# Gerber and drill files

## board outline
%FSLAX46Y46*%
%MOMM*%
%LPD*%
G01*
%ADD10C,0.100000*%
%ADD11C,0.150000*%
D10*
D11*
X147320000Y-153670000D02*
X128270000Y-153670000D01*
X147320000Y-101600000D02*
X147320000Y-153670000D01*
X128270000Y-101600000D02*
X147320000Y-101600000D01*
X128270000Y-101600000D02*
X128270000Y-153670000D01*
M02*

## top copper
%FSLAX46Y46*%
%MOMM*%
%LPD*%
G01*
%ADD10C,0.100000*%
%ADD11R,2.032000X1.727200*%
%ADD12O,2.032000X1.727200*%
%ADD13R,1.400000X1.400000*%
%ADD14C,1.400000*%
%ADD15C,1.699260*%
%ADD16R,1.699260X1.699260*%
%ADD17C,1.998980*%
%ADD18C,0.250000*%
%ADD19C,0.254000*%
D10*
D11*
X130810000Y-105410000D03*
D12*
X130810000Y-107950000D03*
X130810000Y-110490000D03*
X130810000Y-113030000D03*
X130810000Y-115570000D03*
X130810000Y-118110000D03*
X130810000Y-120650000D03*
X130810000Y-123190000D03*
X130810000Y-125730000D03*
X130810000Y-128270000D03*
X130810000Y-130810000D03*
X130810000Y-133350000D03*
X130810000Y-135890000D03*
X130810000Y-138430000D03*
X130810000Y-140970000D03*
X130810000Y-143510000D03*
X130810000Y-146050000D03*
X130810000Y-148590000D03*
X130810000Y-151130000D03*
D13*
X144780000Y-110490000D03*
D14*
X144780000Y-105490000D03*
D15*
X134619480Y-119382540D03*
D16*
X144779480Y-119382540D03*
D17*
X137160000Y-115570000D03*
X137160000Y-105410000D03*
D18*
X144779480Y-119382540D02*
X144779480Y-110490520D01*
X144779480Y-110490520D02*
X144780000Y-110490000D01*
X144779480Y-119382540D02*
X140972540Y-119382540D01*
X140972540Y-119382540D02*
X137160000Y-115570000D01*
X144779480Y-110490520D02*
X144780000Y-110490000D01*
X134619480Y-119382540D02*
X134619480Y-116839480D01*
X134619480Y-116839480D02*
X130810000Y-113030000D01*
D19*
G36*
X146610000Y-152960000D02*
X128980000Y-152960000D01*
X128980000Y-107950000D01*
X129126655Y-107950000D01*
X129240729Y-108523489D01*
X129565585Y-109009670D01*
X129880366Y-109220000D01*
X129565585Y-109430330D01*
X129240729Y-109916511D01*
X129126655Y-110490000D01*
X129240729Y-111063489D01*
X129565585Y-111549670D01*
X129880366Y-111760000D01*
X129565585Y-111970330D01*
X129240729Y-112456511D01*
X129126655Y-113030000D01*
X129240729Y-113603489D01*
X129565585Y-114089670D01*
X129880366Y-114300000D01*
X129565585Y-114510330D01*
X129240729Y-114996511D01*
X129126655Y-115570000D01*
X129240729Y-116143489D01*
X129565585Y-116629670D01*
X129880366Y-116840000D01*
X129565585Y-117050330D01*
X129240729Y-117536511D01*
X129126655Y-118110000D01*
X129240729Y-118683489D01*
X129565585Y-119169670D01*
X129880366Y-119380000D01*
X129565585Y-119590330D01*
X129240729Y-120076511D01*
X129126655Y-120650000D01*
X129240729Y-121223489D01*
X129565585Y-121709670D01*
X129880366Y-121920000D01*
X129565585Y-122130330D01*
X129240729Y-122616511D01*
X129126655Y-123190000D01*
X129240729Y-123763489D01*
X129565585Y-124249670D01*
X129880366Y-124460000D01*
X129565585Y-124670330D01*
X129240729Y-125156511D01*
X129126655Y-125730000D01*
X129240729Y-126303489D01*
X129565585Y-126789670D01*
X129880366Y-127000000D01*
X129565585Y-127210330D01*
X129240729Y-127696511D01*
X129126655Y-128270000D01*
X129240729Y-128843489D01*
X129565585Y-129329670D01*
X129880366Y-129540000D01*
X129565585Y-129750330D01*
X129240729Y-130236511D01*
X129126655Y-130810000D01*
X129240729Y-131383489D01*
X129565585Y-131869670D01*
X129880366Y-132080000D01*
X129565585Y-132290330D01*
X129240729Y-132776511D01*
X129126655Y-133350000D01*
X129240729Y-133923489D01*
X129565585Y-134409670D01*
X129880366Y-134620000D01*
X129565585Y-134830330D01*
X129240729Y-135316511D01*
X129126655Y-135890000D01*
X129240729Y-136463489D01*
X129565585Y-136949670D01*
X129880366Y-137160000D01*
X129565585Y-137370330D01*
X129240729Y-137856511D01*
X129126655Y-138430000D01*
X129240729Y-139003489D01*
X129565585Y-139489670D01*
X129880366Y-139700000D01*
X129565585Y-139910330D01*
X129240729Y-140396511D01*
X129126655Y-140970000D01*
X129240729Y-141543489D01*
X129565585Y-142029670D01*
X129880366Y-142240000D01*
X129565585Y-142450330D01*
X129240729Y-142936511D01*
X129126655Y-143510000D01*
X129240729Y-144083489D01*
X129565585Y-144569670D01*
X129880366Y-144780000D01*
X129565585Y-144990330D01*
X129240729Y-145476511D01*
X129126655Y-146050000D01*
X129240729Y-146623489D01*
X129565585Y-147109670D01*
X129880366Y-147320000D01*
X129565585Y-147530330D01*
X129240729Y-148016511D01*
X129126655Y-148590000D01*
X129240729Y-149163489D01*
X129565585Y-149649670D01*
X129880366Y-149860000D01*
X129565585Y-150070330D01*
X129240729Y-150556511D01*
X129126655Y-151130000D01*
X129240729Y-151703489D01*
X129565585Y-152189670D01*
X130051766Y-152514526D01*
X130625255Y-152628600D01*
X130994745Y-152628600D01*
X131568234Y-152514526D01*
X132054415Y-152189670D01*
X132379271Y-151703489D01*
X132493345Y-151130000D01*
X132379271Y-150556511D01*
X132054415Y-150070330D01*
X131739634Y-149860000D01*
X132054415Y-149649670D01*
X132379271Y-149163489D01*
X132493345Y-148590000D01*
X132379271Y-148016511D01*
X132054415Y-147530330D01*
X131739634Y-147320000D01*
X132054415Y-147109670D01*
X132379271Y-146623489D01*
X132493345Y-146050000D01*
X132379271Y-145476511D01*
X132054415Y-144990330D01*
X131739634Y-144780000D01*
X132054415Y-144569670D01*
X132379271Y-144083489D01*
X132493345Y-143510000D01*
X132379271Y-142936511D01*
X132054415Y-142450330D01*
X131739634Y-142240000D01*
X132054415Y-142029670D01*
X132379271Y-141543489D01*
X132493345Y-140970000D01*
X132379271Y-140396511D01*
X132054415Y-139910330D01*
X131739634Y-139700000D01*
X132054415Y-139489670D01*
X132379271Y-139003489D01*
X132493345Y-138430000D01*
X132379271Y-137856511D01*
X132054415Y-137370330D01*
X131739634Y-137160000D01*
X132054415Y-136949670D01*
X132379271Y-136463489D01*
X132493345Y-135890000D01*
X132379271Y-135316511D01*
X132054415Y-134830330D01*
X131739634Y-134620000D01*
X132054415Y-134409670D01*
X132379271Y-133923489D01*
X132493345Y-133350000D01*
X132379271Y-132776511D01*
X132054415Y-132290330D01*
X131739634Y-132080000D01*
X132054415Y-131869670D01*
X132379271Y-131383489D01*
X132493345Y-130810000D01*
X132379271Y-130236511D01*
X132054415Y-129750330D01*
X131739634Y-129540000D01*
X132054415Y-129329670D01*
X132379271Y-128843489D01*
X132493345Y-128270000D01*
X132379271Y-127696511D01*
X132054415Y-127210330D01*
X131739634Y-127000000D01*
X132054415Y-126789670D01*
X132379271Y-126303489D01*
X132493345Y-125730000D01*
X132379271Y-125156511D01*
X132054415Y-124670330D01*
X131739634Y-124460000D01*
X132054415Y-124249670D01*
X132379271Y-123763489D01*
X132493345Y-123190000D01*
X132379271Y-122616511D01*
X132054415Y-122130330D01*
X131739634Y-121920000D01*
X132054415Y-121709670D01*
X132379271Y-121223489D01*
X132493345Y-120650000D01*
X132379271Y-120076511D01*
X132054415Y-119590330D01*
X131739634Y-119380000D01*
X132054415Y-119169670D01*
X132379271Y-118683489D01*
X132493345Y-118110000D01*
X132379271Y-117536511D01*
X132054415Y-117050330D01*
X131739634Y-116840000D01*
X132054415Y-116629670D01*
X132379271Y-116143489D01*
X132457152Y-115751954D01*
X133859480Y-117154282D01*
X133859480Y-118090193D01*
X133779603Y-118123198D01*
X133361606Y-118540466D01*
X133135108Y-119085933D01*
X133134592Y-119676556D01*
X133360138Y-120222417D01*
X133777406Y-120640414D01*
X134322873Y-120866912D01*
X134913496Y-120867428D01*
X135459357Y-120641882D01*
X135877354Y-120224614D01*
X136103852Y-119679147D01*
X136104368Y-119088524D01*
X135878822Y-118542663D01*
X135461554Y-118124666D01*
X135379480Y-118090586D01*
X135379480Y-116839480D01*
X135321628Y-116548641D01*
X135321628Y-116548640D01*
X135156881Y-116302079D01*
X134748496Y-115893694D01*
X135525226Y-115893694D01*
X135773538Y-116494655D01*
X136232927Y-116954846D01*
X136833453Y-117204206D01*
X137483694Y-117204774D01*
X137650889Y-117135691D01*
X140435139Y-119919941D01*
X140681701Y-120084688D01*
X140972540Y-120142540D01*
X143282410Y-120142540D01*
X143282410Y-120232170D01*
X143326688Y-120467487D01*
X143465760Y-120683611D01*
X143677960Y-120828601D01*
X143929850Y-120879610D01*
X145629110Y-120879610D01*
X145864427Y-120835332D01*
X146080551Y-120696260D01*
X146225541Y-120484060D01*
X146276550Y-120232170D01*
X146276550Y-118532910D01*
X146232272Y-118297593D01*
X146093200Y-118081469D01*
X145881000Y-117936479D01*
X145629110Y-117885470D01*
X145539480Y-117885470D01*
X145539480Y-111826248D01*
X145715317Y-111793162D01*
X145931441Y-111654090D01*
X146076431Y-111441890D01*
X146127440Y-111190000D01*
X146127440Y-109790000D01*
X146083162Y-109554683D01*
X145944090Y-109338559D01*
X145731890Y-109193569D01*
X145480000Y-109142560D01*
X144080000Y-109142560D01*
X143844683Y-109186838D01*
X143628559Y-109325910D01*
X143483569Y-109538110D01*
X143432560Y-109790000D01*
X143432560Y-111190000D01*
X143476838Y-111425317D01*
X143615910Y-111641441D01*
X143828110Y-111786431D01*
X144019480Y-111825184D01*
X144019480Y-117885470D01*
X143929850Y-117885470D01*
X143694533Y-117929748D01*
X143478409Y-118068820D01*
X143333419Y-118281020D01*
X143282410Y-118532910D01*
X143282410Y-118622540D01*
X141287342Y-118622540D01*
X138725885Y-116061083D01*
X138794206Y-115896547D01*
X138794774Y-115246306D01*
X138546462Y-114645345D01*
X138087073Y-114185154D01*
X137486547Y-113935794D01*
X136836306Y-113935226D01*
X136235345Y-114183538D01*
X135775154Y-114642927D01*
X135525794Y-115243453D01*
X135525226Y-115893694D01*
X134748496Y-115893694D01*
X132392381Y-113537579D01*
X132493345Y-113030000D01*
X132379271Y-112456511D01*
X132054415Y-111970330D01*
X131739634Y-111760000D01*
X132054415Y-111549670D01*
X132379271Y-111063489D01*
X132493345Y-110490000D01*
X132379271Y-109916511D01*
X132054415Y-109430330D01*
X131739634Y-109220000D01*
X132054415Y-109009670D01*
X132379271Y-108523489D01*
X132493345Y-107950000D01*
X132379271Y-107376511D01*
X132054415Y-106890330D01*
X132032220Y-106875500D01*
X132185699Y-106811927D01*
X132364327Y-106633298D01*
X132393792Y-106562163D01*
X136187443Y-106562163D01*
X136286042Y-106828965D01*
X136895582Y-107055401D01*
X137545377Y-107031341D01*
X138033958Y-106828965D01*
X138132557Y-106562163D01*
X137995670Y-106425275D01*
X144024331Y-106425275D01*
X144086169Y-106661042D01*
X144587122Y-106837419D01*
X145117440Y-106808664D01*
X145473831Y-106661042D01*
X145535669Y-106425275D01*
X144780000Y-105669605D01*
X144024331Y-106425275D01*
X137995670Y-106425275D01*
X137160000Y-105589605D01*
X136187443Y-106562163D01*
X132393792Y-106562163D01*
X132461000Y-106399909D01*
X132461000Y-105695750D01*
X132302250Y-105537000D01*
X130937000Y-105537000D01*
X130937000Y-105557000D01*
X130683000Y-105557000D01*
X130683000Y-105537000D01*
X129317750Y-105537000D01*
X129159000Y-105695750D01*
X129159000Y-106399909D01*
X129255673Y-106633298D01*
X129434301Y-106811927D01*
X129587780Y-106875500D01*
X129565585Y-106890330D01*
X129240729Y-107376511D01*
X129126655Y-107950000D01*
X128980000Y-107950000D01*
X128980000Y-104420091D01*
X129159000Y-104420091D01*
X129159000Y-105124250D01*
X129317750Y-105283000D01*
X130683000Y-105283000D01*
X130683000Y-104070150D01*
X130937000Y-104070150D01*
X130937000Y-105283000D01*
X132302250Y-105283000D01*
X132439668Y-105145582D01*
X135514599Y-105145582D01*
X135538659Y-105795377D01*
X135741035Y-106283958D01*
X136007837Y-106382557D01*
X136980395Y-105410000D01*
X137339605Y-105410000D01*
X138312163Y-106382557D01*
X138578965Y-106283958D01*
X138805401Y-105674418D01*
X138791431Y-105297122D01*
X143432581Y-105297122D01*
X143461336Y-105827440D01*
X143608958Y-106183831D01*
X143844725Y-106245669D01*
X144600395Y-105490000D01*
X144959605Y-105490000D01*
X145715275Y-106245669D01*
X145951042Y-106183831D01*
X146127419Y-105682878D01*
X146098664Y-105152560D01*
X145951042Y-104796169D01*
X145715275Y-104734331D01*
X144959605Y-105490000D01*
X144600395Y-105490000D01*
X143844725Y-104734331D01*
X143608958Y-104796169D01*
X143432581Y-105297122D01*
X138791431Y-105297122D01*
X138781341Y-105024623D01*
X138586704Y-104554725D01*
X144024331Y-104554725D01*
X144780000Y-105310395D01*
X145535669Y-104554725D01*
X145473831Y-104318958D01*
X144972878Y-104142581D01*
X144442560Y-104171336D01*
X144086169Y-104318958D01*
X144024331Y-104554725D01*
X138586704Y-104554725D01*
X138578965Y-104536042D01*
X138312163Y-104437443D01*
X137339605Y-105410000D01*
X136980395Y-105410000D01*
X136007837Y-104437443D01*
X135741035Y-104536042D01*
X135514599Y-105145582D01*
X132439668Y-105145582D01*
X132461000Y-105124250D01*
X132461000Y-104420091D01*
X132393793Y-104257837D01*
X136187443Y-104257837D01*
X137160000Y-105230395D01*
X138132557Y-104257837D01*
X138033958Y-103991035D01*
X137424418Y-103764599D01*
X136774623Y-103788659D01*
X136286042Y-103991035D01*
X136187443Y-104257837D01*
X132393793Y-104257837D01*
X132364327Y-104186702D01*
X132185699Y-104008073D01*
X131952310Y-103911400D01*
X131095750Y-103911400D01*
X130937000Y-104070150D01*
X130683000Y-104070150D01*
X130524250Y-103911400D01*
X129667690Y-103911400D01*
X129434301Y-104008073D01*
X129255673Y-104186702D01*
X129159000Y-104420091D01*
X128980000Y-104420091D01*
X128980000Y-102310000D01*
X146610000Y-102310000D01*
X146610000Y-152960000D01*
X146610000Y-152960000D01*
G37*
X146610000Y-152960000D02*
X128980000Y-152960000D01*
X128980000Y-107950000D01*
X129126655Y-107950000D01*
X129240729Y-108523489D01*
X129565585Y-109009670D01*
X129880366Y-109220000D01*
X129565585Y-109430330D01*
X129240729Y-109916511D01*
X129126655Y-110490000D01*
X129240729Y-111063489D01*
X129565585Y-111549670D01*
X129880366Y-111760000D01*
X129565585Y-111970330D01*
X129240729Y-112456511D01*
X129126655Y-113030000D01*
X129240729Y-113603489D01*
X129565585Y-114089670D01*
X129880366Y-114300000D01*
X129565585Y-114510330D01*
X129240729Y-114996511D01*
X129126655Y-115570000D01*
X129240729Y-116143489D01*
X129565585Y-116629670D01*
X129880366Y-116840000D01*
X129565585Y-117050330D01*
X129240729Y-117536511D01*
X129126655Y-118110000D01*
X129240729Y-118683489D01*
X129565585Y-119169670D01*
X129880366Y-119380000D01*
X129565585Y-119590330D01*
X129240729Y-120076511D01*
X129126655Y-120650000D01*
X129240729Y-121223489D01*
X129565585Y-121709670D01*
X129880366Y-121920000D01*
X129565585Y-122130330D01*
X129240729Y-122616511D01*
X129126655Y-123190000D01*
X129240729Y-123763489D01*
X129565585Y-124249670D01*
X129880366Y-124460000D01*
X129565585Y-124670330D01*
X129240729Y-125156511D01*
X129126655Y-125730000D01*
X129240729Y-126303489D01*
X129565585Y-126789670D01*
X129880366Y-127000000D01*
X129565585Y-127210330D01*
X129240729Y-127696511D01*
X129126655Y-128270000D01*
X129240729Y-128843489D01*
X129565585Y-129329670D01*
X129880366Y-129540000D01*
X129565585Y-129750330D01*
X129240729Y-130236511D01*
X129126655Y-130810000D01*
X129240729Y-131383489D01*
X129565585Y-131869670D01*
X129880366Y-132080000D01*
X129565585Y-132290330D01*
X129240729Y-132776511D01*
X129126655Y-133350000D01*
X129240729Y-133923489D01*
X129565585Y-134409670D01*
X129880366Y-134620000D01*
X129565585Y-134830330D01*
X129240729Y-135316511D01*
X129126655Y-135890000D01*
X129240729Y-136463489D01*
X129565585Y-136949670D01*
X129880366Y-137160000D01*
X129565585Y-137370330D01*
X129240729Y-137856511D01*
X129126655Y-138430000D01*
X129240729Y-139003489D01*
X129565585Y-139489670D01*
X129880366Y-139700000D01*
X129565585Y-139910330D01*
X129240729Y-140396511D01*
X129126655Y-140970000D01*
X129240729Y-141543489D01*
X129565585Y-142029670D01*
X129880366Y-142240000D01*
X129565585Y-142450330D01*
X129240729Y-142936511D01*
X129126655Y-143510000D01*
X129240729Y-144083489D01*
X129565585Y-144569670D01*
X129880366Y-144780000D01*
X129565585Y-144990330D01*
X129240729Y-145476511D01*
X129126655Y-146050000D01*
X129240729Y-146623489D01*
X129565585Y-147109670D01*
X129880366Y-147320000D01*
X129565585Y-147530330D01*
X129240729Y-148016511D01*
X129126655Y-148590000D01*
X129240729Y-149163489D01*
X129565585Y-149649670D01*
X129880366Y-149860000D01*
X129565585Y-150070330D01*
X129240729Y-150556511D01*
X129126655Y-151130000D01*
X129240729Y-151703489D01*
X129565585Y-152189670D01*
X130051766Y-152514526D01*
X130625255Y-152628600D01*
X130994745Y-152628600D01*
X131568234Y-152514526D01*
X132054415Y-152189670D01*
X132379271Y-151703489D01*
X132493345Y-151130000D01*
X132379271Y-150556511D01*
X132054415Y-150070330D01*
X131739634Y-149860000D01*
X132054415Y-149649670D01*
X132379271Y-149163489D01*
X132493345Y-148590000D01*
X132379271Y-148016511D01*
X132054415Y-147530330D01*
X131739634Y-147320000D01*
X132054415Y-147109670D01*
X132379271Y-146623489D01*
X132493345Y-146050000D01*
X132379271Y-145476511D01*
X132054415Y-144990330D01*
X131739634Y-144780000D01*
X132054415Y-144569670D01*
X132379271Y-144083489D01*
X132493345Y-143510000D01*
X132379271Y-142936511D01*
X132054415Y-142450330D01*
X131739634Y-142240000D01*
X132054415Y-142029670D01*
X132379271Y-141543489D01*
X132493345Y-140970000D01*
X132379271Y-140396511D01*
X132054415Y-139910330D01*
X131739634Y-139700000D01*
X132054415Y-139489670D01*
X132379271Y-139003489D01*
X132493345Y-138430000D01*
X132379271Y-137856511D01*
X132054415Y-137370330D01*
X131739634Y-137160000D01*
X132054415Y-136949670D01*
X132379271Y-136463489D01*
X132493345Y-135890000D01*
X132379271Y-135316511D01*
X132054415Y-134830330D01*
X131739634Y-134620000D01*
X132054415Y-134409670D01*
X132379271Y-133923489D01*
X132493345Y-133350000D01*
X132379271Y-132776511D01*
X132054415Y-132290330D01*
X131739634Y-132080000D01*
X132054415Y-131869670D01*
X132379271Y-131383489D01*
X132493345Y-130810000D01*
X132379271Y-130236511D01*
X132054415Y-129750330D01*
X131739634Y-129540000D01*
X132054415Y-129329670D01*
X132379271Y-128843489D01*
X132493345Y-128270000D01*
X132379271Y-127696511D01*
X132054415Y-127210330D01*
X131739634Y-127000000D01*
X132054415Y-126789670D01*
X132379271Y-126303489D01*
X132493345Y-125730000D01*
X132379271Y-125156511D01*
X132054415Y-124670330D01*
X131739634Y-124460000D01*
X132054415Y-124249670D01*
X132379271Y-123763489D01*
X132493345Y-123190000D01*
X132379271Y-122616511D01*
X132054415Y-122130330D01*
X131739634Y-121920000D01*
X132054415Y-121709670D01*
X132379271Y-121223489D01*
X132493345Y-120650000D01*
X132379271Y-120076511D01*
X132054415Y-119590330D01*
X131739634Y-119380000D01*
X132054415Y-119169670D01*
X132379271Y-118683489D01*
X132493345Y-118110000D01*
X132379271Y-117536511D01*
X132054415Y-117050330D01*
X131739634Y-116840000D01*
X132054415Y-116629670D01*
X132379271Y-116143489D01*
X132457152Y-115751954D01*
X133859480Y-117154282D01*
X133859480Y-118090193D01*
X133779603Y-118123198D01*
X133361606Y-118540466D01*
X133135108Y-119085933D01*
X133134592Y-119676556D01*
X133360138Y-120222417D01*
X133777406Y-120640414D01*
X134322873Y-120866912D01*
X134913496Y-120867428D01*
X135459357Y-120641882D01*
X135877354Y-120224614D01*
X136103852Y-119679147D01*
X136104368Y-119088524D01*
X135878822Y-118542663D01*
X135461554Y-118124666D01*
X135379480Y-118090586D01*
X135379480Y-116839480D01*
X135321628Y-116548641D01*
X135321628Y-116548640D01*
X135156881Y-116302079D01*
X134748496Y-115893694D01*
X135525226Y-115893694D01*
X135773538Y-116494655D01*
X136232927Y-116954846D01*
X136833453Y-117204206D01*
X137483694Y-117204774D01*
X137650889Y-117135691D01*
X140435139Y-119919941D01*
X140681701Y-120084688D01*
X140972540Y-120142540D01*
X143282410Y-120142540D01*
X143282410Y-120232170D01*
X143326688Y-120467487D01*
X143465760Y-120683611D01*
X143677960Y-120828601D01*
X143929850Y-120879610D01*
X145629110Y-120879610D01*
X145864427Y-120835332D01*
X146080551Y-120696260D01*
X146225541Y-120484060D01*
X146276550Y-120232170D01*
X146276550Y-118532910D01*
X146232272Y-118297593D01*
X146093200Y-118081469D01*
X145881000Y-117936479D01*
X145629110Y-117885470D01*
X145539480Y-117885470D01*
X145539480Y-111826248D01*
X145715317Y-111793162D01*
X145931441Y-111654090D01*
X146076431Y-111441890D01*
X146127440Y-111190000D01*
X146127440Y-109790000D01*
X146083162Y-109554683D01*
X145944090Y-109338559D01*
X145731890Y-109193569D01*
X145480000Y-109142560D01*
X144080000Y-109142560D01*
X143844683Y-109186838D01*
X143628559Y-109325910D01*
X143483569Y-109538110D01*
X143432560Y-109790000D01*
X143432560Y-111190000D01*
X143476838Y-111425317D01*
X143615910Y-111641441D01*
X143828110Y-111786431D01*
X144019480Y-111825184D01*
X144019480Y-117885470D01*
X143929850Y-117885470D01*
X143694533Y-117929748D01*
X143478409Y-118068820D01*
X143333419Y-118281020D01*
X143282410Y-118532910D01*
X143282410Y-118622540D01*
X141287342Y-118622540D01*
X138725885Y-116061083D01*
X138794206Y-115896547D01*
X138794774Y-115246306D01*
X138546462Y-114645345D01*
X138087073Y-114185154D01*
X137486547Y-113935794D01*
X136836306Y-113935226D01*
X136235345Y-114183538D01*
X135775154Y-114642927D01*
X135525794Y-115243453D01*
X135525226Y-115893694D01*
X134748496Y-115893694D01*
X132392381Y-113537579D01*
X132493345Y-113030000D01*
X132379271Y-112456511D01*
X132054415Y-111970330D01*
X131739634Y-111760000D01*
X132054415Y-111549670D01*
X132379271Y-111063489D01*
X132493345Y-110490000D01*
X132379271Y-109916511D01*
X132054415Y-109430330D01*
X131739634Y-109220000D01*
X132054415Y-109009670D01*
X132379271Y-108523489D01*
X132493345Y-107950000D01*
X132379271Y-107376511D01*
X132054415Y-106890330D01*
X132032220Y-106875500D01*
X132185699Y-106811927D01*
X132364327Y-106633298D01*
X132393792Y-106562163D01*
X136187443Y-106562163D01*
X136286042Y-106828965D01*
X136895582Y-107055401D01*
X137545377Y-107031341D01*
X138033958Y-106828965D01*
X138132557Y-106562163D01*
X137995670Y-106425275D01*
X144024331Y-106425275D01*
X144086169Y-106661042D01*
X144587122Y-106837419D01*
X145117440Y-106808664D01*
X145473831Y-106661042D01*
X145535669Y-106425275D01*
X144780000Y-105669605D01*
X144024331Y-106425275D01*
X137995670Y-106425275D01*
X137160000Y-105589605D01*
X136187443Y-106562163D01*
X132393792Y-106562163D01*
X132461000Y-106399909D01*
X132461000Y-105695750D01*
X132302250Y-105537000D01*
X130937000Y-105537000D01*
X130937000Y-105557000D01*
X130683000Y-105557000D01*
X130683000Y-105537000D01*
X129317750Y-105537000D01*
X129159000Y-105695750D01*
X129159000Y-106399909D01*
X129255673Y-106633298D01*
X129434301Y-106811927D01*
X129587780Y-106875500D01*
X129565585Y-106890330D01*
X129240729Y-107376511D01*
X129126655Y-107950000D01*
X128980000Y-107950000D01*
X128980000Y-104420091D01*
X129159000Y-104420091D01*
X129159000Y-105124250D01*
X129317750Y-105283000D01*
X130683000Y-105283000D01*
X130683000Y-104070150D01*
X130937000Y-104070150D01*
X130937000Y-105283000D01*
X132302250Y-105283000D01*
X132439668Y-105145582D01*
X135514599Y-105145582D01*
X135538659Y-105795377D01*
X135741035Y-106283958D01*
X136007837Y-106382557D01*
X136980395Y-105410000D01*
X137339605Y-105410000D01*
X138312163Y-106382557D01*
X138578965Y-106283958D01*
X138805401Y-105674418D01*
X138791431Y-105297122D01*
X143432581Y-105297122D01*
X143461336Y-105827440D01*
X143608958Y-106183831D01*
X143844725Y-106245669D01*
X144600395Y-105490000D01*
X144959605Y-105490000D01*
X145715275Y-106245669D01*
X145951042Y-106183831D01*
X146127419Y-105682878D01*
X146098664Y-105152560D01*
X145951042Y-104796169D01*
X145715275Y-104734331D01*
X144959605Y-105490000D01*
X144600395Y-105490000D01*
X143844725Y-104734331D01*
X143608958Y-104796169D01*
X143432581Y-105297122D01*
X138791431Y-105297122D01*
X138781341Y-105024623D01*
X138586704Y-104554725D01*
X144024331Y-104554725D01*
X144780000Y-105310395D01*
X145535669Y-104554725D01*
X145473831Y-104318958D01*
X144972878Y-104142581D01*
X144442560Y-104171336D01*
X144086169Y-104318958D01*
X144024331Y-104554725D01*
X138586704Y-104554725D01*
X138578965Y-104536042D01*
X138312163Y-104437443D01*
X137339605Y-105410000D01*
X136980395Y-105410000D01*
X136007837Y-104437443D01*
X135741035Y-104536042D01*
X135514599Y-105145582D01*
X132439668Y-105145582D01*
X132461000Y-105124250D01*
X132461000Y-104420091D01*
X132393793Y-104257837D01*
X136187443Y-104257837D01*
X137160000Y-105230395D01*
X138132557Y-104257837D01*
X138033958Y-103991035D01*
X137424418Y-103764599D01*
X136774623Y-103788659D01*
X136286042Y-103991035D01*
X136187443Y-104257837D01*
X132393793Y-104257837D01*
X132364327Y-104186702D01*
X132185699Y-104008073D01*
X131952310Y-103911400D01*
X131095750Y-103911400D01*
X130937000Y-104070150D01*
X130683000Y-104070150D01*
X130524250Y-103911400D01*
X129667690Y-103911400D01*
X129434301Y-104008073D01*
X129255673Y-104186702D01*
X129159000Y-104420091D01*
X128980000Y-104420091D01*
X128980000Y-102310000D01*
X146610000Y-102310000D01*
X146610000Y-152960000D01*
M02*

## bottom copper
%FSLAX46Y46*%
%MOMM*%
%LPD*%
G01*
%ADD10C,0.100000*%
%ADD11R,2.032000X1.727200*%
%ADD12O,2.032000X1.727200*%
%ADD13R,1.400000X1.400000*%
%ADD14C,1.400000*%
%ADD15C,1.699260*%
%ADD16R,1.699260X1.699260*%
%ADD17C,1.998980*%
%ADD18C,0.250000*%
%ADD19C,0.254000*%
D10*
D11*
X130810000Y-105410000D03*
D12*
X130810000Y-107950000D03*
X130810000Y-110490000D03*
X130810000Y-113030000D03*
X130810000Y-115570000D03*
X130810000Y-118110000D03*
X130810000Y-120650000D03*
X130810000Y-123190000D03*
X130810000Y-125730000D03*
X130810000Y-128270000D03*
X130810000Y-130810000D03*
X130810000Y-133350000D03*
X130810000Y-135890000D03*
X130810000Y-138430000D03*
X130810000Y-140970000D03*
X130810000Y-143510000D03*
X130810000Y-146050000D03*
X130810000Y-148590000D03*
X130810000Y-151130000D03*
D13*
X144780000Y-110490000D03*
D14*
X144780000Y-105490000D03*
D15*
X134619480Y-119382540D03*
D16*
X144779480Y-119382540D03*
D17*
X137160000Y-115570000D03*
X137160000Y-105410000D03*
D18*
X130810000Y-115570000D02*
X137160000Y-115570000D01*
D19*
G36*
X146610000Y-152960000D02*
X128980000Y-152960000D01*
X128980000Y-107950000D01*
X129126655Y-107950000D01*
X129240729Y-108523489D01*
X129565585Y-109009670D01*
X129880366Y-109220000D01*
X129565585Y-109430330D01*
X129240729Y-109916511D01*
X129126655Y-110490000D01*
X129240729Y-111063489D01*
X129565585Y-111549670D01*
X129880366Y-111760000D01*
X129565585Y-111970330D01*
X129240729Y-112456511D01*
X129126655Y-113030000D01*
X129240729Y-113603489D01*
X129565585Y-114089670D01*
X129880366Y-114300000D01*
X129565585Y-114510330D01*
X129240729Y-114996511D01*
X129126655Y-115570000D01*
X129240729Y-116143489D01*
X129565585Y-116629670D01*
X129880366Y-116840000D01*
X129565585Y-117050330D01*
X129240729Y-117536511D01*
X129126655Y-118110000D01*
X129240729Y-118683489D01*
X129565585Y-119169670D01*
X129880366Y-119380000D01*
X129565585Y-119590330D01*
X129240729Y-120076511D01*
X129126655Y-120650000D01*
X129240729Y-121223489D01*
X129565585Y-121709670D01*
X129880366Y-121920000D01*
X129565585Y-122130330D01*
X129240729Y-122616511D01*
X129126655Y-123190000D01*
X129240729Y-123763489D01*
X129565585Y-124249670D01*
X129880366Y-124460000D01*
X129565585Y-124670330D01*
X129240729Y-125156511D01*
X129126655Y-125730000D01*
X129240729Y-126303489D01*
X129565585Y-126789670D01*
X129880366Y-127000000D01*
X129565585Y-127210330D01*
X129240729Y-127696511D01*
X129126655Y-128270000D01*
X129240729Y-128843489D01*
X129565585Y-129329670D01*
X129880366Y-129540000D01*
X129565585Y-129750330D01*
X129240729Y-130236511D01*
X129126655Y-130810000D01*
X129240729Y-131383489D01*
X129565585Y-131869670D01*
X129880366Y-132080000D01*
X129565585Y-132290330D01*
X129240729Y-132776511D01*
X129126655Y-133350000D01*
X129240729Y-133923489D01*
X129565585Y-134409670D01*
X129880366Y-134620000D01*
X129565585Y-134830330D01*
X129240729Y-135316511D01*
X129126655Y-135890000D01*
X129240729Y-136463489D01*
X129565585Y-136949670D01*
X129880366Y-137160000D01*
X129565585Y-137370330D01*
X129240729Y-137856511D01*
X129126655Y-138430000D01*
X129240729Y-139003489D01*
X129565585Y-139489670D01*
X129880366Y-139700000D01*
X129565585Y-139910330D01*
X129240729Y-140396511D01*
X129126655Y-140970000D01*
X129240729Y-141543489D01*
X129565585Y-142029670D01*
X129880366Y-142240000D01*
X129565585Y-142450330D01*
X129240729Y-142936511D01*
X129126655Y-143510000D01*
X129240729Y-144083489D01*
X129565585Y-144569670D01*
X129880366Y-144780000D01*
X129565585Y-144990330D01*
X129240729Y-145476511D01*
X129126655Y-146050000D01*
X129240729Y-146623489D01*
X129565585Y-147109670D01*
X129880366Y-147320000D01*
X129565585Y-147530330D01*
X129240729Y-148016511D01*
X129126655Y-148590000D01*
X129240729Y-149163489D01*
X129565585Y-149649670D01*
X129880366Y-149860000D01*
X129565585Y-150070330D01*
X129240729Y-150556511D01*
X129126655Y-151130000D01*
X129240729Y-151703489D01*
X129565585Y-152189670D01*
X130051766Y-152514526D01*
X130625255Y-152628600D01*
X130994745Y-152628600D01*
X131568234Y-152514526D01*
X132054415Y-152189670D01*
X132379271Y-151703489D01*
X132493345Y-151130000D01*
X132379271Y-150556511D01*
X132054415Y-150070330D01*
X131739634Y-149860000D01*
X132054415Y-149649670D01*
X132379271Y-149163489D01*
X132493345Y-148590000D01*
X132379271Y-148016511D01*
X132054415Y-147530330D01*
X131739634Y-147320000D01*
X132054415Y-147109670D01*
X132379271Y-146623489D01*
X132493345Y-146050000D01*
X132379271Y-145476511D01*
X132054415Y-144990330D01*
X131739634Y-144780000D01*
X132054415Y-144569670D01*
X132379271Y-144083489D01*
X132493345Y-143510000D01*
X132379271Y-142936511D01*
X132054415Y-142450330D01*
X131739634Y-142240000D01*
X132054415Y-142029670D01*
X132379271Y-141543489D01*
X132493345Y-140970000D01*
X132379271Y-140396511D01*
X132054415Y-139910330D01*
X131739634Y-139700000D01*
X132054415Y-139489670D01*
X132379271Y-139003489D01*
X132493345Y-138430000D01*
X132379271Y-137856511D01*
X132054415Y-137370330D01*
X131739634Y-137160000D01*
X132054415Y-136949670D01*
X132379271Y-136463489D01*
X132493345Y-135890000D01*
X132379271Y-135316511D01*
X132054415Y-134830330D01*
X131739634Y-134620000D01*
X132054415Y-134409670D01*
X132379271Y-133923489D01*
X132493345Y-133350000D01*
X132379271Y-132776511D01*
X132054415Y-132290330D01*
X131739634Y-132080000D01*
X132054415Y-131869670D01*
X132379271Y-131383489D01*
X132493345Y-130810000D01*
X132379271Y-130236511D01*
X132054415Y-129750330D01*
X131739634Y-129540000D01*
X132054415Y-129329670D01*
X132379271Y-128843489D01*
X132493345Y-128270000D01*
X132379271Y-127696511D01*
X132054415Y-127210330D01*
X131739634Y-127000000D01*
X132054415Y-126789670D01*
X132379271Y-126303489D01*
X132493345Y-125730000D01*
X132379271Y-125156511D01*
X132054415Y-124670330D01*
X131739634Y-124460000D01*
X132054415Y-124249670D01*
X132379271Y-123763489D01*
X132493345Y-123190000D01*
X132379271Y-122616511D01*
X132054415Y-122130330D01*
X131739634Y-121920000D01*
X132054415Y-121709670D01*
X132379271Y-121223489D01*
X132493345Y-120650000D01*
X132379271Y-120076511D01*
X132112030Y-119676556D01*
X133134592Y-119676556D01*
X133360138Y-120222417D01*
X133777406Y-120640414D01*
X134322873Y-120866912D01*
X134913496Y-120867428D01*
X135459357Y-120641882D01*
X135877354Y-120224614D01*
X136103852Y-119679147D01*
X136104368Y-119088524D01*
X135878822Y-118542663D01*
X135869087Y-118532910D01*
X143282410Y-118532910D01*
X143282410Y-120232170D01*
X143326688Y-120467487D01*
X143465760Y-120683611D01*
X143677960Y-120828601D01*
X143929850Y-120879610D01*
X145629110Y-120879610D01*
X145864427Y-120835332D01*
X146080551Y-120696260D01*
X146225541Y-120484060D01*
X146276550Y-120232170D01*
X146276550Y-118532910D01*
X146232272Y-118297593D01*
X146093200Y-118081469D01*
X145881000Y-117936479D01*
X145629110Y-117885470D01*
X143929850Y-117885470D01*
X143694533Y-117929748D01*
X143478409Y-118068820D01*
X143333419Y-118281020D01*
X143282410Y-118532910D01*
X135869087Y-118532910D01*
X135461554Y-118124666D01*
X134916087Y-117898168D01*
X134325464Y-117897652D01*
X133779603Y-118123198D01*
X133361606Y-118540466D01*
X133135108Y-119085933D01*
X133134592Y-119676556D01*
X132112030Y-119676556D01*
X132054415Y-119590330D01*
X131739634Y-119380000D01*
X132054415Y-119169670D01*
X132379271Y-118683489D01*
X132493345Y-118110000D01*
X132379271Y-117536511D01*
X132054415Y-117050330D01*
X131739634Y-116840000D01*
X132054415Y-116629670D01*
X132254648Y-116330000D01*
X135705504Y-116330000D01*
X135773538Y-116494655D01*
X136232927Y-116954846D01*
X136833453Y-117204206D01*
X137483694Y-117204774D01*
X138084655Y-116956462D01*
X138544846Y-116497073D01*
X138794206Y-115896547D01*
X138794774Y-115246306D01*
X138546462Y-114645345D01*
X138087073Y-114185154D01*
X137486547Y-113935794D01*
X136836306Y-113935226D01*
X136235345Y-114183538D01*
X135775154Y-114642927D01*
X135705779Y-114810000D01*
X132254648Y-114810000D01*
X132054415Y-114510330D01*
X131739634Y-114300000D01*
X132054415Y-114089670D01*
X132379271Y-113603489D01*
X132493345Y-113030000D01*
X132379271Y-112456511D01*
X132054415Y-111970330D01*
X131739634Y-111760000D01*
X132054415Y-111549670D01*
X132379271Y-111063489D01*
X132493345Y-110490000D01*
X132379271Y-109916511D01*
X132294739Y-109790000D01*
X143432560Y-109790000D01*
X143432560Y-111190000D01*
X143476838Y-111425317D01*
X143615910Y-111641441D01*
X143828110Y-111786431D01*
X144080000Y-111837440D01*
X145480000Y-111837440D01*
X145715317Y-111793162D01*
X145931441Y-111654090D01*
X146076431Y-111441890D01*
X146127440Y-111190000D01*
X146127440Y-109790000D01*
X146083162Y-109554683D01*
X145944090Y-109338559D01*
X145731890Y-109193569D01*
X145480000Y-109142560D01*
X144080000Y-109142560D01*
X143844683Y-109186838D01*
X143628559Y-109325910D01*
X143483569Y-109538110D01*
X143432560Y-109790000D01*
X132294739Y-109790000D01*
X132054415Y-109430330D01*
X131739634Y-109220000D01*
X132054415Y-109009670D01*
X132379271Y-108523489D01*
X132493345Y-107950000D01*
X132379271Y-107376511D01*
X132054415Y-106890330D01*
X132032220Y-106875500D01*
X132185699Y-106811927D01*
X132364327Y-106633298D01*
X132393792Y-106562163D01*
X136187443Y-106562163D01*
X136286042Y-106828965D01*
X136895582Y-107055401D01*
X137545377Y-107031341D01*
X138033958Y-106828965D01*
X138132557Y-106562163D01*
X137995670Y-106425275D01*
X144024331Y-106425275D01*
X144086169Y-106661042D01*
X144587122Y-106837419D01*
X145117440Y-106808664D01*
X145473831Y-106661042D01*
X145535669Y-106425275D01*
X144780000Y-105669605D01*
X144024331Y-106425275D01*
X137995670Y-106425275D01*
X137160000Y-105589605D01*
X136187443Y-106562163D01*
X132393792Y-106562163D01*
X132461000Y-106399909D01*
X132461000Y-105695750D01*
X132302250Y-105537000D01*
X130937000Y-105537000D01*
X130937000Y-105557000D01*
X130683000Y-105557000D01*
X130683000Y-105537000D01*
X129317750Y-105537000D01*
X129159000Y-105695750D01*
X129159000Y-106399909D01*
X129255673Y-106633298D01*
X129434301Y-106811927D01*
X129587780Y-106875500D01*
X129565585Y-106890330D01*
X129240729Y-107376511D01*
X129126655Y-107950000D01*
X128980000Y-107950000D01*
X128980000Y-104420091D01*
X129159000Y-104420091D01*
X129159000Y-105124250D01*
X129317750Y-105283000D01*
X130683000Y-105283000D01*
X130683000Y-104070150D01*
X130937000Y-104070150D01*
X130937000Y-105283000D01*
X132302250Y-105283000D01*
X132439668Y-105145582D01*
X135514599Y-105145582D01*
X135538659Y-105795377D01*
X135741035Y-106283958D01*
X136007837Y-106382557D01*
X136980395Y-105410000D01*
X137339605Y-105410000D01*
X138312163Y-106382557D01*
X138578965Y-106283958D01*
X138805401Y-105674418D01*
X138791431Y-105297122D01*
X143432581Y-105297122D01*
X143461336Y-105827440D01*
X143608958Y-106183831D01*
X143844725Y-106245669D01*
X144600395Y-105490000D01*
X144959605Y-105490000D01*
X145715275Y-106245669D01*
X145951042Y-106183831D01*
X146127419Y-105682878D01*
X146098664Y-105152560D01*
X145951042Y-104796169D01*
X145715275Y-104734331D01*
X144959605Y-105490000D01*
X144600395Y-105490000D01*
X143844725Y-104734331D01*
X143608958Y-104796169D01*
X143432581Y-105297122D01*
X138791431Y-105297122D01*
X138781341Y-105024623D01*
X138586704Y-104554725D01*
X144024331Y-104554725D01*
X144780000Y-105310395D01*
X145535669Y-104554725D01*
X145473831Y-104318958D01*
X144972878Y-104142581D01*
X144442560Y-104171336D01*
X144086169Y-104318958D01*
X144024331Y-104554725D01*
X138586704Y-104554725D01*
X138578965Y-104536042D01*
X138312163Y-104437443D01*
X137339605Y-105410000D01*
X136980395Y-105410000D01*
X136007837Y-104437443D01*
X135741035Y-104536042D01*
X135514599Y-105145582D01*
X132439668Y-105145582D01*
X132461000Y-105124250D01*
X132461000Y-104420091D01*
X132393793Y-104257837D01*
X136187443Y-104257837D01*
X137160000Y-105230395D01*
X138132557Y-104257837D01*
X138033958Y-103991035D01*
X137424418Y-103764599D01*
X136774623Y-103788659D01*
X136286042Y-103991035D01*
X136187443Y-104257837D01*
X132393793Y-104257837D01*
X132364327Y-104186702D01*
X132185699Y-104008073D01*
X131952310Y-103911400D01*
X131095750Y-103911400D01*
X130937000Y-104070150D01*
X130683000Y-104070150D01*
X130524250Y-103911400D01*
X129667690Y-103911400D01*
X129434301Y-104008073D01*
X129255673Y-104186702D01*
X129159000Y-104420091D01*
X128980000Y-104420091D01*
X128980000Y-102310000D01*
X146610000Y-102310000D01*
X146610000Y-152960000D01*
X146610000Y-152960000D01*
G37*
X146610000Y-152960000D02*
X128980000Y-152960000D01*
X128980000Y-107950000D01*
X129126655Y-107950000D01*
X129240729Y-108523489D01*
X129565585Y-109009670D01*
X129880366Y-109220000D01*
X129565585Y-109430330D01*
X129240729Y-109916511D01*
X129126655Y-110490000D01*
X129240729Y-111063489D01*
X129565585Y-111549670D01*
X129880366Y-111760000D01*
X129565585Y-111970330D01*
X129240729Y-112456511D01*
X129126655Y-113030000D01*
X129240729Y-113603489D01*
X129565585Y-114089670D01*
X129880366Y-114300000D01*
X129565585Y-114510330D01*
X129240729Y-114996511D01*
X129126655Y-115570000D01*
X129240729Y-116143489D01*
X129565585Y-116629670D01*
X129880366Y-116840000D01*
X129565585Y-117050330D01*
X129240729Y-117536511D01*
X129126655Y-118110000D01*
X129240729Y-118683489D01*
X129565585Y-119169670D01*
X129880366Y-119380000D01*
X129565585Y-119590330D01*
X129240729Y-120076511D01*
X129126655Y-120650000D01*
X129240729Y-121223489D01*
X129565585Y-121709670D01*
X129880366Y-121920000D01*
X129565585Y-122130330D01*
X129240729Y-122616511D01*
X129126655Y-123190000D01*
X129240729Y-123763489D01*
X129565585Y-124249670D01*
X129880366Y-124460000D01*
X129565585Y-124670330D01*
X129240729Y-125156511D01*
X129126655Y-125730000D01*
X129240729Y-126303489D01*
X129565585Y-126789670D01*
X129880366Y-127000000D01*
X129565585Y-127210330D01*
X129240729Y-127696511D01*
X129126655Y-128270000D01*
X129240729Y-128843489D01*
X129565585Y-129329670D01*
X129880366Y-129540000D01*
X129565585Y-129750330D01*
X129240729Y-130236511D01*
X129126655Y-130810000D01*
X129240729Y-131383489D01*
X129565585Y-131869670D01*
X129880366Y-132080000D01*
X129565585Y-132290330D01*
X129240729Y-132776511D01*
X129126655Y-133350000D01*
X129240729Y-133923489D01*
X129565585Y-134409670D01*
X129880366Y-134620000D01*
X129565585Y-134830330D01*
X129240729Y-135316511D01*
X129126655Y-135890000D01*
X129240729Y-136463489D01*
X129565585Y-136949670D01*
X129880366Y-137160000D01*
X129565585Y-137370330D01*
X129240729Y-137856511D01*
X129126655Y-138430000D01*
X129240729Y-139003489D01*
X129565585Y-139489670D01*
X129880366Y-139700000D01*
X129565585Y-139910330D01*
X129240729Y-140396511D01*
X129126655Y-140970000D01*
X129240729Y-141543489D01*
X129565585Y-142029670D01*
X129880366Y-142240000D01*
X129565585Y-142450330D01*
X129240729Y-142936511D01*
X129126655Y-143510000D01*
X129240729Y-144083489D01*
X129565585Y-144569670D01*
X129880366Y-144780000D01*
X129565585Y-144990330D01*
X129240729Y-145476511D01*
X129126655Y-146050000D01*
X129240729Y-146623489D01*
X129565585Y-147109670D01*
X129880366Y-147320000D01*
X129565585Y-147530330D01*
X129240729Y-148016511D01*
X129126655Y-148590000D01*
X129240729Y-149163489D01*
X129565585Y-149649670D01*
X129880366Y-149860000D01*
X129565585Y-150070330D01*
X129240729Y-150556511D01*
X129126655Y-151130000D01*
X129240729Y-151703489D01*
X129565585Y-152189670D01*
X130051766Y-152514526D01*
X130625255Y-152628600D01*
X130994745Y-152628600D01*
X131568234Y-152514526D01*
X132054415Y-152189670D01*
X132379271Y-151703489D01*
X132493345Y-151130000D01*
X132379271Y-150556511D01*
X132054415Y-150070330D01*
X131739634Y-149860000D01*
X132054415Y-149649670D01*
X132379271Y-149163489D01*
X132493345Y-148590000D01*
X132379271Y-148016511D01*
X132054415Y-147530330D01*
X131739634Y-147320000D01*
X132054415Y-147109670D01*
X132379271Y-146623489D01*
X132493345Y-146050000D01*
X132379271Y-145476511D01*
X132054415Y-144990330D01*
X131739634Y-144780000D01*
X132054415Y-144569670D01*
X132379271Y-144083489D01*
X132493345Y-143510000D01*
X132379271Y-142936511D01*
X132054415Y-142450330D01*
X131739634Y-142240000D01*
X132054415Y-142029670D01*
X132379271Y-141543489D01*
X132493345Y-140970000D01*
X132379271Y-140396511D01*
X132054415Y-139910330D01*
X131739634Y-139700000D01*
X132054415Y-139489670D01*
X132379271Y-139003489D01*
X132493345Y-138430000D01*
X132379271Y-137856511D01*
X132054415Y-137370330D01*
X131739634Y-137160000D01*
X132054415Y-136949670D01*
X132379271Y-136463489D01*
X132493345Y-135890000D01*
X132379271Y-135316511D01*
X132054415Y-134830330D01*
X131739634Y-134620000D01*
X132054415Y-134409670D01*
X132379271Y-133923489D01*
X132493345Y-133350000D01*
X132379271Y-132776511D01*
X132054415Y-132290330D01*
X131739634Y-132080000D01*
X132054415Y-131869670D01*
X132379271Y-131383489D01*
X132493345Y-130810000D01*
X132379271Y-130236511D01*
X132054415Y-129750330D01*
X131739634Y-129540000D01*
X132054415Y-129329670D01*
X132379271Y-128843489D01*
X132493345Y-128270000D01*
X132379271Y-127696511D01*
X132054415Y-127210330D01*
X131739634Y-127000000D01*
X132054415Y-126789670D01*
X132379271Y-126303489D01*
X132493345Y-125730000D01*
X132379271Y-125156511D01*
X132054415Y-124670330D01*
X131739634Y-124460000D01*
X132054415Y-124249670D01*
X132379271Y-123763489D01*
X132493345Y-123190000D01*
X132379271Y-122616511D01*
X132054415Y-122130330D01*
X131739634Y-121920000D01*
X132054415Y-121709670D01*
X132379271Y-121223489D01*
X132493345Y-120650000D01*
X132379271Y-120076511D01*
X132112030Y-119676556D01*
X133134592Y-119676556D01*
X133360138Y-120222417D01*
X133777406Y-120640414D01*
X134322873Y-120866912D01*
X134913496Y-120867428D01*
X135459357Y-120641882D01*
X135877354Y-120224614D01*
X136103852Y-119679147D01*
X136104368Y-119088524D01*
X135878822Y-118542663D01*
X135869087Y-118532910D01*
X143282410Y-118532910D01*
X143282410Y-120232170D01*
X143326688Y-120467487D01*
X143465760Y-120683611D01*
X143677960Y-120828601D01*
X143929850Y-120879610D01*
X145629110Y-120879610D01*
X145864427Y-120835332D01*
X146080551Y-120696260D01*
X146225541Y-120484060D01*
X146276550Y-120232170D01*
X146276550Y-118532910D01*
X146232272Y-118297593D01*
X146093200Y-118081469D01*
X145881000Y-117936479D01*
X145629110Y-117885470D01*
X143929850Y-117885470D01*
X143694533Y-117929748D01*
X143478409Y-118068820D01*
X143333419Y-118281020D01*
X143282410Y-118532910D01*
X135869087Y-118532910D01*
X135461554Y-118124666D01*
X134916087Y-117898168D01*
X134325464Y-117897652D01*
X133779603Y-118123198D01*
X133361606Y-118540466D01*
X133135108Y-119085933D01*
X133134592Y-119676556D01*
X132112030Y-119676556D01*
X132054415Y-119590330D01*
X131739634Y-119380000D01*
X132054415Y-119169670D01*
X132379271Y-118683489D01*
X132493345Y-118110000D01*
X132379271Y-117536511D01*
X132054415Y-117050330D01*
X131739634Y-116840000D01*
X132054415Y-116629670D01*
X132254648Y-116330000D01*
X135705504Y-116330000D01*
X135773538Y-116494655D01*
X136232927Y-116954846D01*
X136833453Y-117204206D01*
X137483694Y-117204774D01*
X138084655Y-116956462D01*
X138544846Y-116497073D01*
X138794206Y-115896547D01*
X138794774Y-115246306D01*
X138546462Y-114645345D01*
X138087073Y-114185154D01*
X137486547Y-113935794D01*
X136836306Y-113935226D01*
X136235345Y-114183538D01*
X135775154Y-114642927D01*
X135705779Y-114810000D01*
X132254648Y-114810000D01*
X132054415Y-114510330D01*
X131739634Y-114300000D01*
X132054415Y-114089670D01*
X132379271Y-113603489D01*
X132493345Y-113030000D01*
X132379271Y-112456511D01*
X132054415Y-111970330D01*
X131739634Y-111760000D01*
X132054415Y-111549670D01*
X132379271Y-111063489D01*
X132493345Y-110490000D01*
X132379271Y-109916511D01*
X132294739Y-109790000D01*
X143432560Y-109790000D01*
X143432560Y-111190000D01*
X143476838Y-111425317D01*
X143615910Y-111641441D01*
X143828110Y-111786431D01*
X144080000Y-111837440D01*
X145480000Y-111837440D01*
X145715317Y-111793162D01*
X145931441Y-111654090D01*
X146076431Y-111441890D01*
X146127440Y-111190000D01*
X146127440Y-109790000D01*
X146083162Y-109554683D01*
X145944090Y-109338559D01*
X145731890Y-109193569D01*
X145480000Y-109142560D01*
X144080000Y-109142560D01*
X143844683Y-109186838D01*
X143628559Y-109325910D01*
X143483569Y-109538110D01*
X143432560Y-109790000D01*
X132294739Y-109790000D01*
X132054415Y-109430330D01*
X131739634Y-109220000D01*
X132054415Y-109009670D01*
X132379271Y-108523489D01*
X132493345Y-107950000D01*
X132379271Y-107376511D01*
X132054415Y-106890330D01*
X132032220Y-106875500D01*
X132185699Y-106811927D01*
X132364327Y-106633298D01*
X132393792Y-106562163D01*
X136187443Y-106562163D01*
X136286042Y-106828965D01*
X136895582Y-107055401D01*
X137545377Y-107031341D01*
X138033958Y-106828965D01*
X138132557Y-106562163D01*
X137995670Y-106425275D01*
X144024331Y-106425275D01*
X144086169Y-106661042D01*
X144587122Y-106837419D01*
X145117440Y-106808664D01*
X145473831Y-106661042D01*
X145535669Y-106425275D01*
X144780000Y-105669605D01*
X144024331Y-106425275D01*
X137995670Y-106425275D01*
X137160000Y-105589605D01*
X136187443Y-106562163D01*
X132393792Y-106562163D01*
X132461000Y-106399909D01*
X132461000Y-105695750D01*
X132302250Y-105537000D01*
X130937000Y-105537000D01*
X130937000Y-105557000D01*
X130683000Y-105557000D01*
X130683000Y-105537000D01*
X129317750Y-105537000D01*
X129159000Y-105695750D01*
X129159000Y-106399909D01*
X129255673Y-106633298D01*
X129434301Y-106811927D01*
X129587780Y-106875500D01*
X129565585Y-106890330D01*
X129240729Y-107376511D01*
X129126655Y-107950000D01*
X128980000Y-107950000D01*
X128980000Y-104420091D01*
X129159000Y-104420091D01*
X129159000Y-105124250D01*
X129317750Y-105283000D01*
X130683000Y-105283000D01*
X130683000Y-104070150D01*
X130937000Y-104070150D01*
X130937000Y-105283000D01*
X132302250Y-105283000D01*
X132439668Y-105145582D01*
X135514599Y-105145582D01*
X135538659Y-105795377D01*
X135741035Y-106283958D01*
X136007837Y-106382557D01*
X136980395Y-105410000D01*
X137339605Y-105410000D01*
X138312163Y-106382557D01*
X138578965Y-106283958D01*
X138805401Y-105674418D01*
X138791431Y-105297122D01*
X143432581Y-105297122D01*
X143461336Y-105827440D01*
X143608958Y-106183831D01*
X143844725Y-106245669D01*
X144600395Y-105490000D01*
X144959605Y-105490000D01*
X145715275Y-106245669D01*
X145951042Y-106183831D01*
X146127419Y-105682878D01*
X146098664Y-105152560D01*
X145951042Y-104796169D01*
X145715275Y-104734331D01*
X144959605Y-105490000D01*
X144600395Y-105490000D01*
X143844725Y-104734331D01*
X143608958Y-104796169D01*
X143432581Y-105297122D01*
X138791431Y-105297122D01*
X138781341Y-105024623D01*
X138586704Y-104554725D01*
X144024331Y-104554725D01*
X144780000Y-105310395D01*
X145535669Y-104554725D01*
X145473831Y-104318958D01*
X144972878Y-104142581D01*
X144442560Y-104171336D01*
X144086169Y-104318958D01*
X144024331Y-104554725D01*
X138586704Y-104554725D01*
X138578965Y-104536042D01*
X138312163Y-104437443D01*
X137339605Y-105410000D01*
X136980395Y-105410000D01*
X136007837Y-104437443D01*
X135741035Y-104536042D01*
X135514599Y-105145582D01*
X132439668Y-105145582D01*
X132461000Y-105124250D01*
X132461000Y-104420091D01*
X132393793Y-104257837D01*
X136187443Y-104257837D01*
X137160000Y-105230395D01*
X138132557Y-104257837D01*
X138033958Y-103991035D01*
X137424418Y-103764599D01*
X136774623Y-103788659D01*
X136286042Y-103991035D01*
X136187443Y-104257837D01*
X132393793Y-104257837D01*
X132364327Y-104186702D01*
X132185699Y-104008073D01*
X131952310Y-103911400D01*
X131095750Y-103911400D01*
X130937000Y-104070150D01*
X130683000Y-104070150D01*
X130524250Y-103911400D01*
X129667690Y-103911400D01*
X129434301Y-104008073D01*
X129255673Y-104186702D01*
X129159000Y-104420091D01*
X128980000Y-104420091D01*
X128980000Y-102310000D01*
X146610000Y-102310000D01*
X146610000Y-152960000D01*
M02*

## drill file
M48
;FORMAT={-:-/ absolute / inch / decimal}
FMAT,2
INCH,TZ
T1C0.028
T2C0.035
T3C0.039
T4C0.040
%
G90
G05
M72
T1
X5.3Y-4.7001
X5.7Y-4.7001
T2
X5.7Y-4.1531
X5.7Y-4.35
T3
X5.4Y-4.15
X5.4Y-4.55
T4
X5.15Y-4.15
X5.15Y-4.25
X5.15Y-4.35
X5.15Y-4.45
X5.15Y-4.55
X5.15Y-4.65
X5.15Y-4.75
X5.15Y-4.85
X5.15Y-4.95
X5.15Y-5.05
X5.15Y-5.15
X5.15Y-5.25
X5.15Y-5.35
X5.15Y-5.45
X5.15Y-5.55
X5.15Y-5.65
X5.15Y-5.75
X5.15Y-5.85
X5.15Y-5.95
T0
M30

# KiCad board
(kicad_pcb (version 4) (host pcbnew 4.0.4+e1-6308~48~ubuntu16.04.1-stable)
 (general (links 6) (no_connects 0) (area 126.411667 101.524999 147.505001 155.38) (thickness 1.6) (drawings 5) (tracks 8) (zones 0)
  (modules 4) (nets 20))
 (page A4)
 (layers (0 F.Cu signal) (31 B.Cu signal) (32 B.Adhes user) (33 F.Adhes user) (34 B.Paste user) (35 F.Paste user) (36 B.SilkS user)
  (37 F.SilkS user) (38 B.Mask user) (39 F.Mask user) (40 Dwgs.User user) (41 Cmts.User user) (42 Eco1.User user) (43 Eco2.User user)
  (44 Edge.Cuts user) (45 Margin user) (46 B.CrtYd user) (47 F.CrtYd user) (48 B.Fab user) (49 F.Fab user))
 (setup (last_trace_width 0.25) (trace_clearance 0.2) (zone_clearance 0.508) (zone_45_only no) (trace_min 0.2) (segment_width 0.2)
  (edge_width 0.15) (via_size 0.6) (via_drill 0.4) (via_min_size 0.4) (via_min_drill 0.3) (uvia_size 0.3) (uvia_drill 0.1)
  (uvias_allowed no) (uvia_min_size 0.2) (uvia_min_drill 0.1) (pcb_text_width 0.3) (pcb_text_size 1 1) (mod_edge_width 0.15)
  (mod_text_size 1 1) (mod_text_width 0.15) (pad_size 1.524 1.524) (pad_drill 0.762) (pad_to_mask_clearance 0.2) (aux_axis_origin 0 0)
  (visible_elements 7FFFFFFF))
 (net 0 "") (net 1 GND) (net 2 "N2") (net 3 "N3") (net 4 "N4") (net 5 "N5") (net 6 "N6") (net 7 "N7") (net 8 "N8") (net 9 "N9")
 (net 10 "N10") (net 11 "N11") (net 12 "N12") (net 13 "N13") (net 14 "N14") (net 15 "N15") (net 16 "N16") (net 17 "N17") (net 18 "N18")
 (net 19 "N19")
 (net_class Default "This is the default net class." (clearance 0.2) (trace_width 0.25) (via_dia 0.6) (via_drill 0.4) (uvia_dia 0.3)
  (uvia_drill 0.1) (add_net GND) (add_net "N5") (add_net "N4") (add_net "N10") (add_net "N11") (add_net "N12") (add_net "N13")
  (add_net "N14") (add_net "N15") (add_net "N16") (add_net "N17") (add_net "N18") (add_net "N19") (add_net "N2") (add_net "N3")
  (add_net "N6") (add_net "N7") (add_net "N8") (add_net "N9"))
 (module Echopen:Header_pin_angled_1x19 (layer F.Cu) (at 130.81 128.27)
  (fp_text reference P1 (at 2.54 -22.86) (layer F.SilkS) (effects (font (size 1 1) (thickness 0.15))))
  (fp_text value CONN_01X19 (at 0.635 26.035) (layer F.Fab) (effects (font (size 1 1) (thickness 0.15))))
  (pad 1 thru_hole rect (at 0 -22.86 270) (size 1.7272 2.032) (drill 1.016) (layers *.Cu *.Mask F.SilkS) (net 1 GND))
  (pad 2 thru_hole oval (at 0 -20.32 270) (size 1.7272 2.032) (drill 1.016) (layers *.Cu *.Mask F.SilkS) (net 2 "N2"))
  (pad 3 thru_hole oval (at 0 -17.78 270) (size 1.7272 2.032) (drill 1.016) (layers *.Cu *.Mask F.SilkS) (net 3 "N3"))
  (pad 4 thru_hole oval (at 0 -15.24 270) (size 1.7272 2.032) (drill 1.016) (layers *.Cu *.Mask F.SilkS) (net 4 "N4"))
  (pad 5 thru_hole oval (at 0 -12.7 270) (size 1.7272 2.032) (drill 1.016) (layers *.Cu *.Mask F.SilkS) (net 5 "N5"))
  (pad 6 thru_hole oval (at 0 -10.16 270) (size 1.7272 2.032) (drill 1.016) (layers *.Cu *.Mask F.SilkS) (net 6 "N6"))
  (pad 7 thru_hole oval (at 0 -7.62 270) (size 1.7272 2.032) (drill 1.016) (layers *.Cu *.Mask F.SilkS) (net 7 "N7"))
  (pad 8 thru_hole oval (at 0 -5.08 270) (size 1.7272 2.032) (drill 1.016) (layers *.Cu *.Mask F.SilkS) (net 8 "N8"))
  (pad 9 thru_hole oval (at 0 -2.54 270) (size 1.7272 2.032) (drill 1.016) (layers *.Cu *.Mask F.SilkS) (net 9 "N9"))
  (pad 10 thru_hole oval (at 0 0 270) (size 1.7272 2.032) (drill 1.016) (layers *.Cu *.Mask F.SilkS) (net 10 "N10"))
  (pad 11 thru_hole oval (at 0 2.54 270) (size 1.7272 2.032) (drill 1.016) (layers *.Cu *.Mask F.SilkS) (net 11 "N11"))
  (pad 12 thru_hole oval (at 0 5.08 270) (size 1.7272 2.032) (drill 1.016) (layers *.Cu *.Mask F.SilkS) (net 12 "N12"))
  (pad 13 thru_hole oval (at 0 7.62 270) (size 1.7272 2.032) (drill 1.016) (layers *.Cu *.Mask F.SilkS) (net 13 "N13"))
  (pad 14 thru_hole oval (at 0 10.16 270) (size 1.7272 2.032) (drill 1.016) (layers *.Cu *.Mask F.SilkS) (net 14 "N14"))
  (pad 15 thru_hole oval (at 0 12.7 270) (size 1.7272 2.032) (drill 1.016) (layers *.Cu *.Mask F.SilkS) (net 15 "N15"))
  (pad 16 thru_hole oval (at 0 15.24 270) (size 1.7272 2.032) (drill 1.016) (layers *.Cu *.Mask F.SilkS) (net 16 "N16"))
  (pad 17 thru_hole oval (at 0 17.78 270) (size 1.7272 2.032) (drill 1.016) (layers *.Cu *.Mask F.SilkS) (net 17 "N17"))
  (pad 18 thru_hole oval (at 0 20.32 270) (size 1.7272 2.032) (drill 1.016) (layers *.Cu *.Mask F.SilkS) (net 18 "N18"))
  (pad 19 thru_hole oval (at 0 22.86 270) (size 1.7272 2.032) (drill 1.016) (layers *.Cu *.Mask F.SilkS) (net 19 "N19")))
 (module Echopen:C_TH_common (layer F.Cu) (at 144.78 110.49 90)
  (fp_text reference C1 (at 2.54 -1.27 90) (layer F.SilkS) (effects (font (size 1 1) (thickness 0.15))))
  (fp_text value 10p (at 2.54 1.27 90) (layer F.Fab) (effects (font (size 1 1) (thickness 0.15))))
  (pad 1 thru_hole rect (at 0 0 90) (size 1.4 1.4) (drill 0.9) (layers *.Cu *.Mask F.SilkS) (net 5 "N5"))
  (pad 2 thru_hole circle (at 5 0 90) (size 1.4 1.4) (drill 0.9) (layers *.Cu *.Mask F.SilkS) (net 1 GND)))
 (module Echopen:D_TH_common (layer F.Cu) (at 144.78 119.38 180)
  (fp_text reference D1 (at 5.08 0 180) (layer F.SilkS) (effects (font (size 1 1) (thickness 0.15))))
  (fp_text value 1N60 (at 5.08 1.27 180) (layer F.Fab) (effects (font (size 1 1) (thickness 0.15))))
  (pad 2 thru_hole circle (at 10.16052 -0.00254) (size 1.69926 1.69926) (drill 0.70104) (layers *.Cu *.Mask F.SilkS) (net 4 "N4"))
  (pad 1 thru_hole rect (at 0.00052 -0.00254) (size 1.69926 1.69926) (drill 0.70104) (layers *.Cu *.Mask F.SilkS) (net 5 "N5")))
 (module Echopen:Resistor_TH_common (layer F.Cu) (at 137.16 115.57 90)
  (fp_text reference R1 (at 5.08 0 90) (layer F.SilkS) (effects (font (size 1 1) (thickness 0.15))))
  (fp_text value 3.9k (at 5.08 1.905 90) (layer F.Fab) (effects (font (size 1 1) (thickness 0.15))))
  (pad 1 thru_hole circle (at 0 0 90) (size 1.99898 1.99898) (drill 1.00076) (layers *.Cu *.SilkS *.Mask) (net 5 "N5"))
  (pad 2 thru_hole circle (at 10.16 0 90) (size 1.99898 1.99898) (drill 1.00076) (layers *.Cu *.SilkS *.Mask) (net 1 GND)))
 (gr_line (start 147.32 153.67) (end 128.27 153.67) (angle 90) (layer Edge.Cuts) (width 0.15))
 (gr_line (start 147.32 101.6) (end 147.32 153.67) (angle 90) (layer Edge.Cuts) (width 0.15))
 (gr_line (start 128.27 101.6) (end 147.32 101.6) (angle 90) (layer Edge.Cuts) (width 0.15))
 (gr_line (start 128.27 101.6) (end 128.27 153.67) (angle 90) (layer Edge.Cuts) (width 0.15))
 (segment (start 144.77948 119.38254) (end 144.77948 110.49052) (width 0.25) (layer F.Cu) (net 5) (status 20))
 (segment (start 144.77948 110.49052) (end 144.78 110.49) (width 0.25) (layer F.Cu) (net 5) (status 30))
 (segment (start 130.81 115.57) (end 137.16 115.57) (width 0.25) (layer B.Cu) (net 5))
 (segment (start 144.77948 119.38254) (end 140.97254 119.38254) (width 0.25) (layer F.Cu) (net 5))
 (segment (start 140.97254 119.38254) (end 137.16 115.57) (width 0.25) (layer F.Cu) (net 5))
 (segment (start 144.77948 110.49052) (end 144.78 110.49) (width 0.25) (layer F.Cu) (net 5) (status 30))
 (segment (start 134.61948 119.38254) (end 134.61948 116.83948) (width 0.25) (layer F.Cu) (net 4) (status 10))
 (segment (start 134.61948 116.83948) (end 130.81 113.03) (width 0.25) (layer F.Cu) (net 4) (status 20))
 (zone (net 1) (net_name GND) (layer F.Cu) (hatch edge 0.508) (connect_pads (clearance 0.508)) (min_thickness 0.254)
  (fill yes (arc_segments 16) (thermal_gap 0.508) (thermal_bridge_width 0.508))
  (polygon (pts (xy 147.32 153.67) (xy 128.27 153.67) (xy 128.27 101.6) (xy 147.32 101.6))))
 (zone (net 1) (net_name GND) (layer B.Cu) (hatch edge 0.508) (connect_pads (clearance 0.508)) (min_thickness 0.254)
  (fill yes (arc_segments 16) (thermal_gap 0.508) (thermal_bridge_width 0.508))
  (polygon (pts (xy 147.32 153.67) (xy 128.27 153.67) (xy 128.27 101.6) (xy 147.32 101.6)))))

